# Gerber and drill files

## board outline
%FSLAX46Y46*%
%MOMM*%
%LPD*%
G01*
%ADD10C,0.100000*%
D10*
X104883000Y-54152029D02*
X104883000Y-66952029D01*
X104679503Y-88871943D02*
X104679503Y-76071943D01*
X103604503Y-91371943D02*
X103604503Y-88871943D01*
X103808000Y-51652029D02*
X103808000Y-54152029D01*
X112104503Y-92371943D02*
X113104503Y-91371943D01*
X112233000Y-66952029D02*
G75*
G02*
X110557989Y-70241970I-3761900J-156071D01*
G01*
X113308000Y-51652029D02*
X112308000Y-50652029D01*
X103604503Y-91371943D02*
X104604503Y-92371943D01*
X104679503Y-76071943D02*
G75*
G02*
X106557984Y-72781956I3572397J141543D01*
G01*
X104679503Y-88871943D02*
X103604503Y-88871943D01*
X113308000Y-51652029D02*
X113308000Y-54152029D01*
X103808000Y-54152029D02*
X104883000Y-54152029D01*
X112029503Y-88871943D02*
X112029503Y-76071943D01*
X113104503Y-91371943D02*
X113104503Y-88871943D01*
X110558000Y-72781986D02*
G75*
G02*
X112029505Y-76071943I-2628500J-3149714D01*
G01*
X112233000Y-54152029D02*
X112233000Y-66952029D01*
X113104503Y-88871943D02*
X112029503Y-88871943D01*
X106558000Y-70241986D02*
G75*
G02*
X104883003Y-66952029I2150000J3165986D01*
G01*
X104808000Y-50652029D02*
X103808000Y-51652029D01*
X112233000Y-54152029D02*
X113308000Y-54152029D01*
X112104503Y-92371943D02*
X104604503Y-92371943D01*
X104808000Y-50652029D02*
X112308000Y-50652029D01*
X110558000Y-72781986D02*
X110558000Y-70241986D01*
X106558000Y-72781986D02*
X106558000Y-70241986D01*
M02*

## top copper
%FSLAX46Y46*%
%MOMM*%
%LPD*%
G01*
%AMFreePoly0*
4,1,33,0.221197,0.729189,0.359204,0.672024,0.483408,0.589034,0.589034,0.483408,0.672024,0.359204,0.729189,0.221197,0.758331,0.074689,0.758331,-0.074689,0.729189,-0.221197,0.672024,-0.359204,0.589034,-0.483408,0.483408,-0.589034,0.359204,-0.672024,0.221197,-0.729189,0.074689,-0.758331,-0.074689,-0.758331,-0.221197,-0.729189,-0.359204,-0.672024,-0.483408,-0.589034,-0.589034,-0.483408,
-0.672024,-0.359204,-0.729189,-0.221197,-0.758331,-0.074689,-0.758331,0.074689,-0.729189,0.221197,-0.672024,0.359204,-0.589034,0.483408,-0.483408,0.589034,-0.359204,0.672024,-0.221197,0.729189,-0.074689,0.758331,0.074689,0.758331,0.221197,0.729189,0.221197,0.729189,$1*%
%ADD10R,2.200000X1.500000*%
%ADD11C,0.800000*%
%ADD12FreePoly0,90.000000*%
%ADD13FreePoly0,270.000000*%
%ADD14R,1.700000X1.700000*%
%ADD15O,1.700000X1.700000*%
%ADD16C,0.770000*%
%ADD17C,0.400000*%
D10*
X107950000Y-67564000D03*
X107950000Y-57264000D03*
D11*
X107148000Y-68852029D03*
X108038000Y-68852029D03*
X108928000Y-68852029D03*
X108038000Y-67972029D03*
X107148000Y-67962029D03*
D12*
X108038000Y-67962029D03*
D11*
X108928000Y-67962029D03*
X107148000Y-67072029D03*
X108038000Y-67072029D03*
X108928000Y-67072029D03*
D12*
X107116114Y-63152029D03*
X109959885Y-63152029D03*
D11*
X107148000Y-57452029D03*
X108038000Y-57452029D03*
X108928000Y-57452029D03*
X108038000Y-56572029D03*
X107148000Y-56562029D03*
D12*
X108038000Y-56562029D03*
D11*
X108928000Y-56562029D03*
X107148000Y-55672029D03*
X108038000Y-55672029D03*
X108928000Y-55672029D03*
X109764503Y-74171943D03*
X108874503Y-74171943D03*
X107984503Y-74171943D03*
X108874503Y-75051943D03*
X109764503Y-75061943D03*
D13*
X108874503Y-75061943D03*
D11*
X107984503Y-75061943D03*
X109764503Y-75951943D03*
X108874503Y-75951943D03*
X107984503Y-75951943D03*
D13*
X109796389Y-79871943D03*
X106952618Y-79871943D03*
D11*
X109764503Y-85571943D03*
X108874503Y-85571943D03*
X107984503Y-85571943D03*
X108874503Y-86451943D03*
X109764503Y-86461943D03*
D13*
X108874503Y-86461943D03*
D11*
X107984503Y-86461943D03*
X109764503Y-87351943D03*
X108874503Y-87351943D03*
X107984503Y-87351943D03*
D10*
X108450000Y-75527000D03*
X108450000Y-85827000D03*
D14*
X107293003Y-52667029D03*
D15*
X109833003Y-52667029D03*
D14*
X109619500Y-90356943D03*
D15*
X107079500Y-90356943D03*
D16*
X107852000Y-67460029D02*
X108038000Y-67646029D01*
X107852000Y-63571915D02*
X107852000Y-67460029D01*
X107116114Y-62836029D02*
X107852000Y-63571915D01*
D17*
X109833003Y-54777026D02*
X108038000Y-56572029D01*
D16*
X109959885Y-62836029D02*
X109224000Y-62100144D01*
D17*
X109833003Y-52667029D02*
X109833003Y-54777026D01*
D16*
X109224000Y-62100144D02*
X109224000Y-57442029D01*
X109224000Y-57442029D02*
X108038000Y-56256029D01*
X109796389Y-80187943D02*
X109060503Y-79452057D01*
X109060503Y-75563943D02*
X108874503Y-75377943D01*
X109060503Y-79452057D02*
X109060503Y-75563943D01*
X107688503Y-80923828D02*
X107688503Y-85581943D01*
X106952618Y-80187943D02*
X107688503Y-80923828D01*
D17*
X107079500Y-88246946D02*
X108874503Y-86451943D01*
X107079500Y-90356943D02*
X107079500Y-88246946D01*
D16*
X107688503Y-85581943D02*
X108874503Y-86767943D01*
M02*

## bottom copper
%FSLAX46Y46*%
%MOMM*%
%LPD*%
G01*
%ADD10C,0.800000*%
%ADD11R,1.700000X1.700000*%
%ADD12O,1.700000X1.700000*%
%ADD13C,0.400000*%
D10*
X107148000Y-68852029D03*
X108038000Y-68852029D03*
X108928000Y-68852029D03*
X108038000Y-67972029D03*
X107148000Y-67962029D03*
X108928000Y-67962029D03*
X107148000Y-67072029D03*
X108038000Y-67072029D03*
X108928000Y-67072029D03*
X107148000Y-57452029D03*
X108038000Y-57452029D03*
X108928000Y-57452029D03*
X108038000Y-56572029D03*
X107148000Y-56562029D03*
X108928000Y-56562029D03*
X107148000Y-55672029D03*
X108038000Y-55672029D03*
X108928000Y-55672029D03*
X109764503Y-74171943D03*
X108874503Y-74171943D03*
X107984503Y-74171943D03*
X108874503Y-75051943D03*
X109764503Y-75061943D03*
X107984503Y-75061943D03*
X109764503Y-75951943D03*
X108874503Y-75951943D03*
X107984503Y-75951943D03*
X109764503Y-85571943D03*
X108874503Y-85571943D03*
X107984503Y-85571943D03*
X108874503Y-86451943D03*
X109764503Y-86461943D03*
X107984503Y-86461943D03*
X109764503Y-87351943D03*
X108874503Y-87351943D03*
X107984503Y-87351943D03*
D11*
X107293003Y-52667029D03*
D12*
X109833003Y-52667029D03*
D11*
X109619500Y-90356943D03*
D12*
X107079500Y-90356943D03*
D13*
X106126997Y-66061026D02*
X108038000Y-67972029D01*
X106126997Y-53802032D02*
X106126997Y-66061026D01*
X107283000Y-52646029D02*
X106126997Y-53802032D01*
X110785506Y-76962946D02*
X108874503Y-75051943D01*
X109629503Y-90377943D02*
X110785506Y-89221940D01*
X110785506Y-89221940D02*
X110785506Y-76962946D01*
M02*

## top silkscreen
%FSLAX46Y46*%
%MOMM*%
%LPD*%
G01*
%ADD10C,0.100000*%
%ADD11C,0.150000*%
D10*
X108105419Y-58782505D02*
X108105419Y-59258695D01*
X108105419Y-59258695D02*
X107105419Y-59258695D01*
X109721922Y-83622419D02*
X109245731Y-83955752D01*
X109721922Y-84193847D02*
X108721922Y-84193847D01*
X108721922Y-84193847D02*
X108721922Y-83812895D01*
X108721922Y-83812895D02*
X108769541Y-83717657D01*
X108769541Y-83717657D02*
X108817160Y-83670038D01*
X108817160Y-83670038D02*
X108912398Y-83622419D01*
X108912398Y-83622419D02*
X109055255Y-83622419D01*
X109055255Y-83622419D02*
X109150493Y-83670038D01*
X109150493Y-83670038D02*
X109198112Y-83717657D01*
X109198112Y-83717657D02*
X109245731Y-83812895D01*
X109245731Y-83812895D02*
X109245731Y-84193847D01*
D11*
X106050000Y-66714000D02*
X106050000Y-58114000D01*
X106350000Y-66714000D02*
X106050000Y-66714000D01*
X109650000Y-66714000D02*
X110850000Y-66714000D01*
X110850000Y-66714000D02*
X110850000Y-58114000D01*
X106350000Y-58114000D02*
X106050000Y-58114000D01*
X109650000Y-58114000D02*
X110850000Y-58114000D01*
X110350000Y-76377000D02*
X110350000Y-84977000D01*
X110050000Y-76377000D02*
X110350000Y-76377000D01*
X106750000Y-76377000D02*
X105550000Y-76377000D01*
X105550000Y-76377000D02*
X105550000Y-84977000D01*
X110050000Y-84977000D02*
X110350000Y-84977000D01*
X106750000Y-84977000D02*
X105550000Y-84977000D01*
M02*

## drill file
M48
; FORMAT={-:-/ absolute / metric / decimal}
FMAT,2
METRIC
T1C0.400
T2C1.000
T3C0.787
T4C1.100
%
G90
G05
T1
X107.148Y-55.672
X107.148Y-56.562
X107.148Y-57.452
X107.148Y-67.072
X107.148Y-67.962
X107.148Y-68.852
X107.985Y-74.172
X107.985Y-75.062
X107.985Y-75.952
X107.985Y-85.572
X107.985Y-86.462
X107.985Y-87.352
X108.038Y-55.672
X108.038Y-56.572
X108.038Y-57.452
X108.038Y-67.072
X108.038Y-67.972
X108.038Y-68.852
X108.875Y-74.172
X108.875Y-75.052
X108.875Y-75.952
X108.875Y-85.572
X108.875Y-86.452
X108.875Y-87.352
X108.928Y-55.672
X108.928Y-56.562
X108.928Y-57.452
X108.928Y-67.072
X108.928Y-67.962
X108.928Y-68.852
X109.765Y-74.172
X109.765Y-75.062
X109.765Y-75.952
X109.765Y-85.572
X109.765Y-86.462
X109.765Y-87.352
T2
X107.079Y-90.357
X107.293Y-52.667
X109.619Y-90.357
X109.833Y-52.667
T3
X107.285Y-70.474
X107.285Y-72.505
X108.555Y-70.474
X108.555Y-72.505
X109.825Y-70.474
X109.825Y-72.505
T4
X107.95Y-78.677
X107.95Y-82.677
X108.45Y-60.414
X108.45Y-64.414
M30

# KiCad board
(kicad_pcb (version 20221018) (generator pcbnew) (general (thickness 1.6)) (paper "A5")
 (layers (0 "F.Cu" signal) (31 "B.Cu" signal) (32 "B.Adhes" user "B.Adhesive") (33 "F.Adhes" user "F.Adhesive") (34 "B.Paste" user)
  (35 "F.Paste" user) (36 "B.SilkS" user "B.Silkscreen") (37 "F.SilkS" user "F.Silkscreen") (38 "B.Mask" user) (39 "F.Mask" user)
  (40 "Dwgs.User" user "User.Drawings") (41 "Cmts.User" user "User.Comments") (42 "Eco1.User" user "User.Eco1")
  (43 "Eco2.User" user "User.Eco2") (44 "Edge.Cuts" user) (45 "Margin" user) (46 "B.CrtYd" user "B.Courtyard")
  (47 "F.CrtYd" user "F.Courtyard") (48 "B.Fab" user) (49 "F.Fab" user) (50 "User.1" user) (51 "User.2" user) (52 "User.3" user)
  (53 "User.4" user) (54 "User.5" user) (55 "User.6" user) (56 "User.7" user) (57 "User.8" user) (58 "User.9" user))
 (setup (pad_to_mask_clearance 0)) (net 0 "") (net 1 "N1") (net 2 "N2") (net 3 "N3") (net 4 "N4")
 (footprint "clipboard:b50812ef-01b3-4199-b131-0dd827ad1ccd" (layer "F.Cu") (at 110.95 68.339 90)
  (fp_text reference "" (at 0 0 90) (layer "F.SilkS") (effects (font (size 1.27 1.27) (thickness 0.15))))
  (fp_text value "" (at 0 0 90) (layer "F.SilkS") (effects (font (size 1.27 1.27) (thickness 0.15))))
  (fp_line (start 1.625 -4.9) (end 10.225 -4.9) (stroke (width 0.15) (type solid)) (layer "F.SilkS"))
  (fp_line (start 1.625 -4.6) (end 1.625 -4.9) (stroke (width 0.15) (type solid)) (layer "F.SilkS"))
  (fp_line (start 1.625 -1.3) (end 1.625 -0.1) (stroke (width 0.15) (type solid)) (layer "F.SilkS"))
  (fp_line (start 1.625 -0.1) (end 10.225 -0.1) (stroke (width 0.15) (type solid)) (layer "F.SilkS"))
  (fp_line (start 10.225 -4.6) (end 10.225 -4.9) (stroke (width 0.15) (type solid)) (layer "F.SilkS"))
  (fp_line (start 10.225 -1.3) (end 10.225 -0.1) (stroke (width 0.15) (type solid)) (layer "F.SilkS"))
  (pad "" np_thru_hole circle (at 3.925 -2.5 90) (size 1.1 1.1) (drill 1.1) (layers "F&B.Cu" "*.Mask"))
  (pad "" np_thru_hole circle (at 7.925 -2.5 90) (size 1.1 1.1) (drill 1.1) (layers "F&B.Cu" "*.Mask"))
  (pad "1" smd rect (at 0.775 -3 90) (size 1.5 2.2) (layers "F.Cu" "F.Paste" "F.Mask"))
  (pad "2" smd rect (at 11.075 -3 90) (size 1.5 2.2) (layers "F.Cu" "F.Paste" "F.Mask")))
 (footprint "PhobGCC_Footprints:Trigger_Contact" (layer "F.Cu") (at 108.538 63.152029 90)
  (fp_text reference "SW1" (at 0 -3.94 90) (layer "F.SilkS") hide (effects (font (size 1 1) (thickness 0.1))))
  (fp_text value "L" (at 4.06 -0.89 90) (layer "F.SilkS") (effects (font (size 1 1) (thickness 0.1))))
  (pad "1" thru_hole circle (at -5.7 -1.39 90) (size 0.8 0.8) (drill 0.4) (layers "*.Cu" "*.Mask") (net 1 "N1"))
  (pad "1" thru_hole circle (at -5.7 -0.5 90) (size 0.8 0.8) (drill 0.4) (layers "*.Cu" "*.Mask") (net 1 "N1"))
  (pad "1" thru_hole circle (at -5.7 0.39 90) (size 0.8 0.8) (drill 0.4) (layers "*.Cu" "*.Mask") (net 1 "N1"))
  (pad "1" thru_hole circle (at -4.82 -0.5 90) (size 0.8 0.8) (drill 0.4) (layers "*.Cu" "*.Mask") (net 1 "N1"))
  (pad "1" thru_hole circle (at -4.81 -1.39 90) (size 0.8 0.8) (drill 0.4) (layers "*.Cu" "*.Mask") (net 1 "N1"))
  (pad "1" smd custom (at -4.81 -0.5 90) (size 1.524 1.524) (layers "F.Cu" "F.Paste" "F.Mask") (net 1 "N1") (thermal_bridge_angle 45)
   (options (clearance outline) (anchor circle)) (primitives))
  (pad "1" thru_hole circle (at -4.81 0.39 90) (size 0.8 0.8) (drill 0.4) (layers "*.Cu" "*.Mask") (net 1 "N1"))
  (pad "1" thru_hole circle (at -3.92 -1.39 90) (size 0.8 0.8) (drill 0.4) (layers "*.Cu" "*.Mask") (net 1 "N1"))
  (pad "1" thru_hole circle (at -3.92 -0.5 90) (size 0.8 0.8) (drill 0.4) (layers "*.Cu" "*.Mask") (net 1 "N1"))
  (pad "1" thru_hole circle (at -3.92 0.39 90) (size 0.8 0.8) (drill 0.4) (layers "*.Cu" "*.Mask") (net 1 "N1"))
  (pad "1" smd custom (at 0 -1.421886 90) (size 1.524 1.524) (layers "F.Cu" "F.Paste" "F.Mask") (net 1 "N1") (thermal_bridge_angle 45)
   (options (clearance outline) (anchor circle)) (primitives))
  (pad "2" smd custom (at 0 1.421885 90) (size 1.524 1.524) (layers "F.Cu" "F.Paste" "F.Mask") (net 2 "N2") (thermal_bridge_angle 45)
   (options (clearance outline) (anchor circle)) (primitives))
  (pad "2" thru_hole circle (at 5.7 -1.39 90) (size 0.8 0.8) (drill 0.4) (layers "*.Cu" "*.Mask") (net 2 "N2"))
  (pad "2" thru_hole circle (at 5.7 -0.5 90) (size 0.8 0.8) (drill 0.4) (layers "*.Cu" "*.Mask") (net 2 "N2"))
  (pad "2" thru_hole circle (at 5.7 0.39 90) (size 0.8 0.8) (drill 0.4) (layers "*.Cu" "*.Mask") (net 2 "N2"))
  (pad "2" thru_hole circle (at 6.58 -0.5 90) (size 0.8 0.8) (drill 0.4) (layers "*.Cu" "*.Mask") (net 2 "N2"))
  (pad "2" thru_hole circle (at 6.59 -1.39 90) (size 0.8 0.8) (drill 0.4) (layers "*.Cu" "*.Mask") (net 2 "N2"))
  (pad "2" smd custom (at 6.59 -0.5 90) (size 1.524 1.524) (layers "F.Cu" "F.Paste" "F.Mask") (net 2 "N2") (thermal_bridge_angle 45)
   (options (clearance outline) (anchor circle)) (primitives))
  (pad "2" thru_hole circle (at 6.59 0.39 90) (size 0.8 0.8) (drill 0.4) (layers "*.Cu" "*.Mask") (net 2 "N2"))
  (pad "2" thru_hole circle (at 7.48 -1.39 90) (size 0.8 0.8) (drill 0.4) (layers "*.Cu" "*.Mask") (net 2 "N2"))
  (pad "2" thru_hole circle (at 7.48 -0.5 90) (size 0.8 0.8) (drill 0.4) (layers "*.Cu" "*.Mask") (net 2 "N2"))
  (pad "2" thru_hole circle (at 7.48 0.39 90) (size 0.8 0.8) (drill 0.4) (layers "*.Cu" "*.Mask") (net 2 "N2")))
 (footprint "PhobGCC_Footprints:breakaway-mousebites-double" (layer "F.Cu") (at 108.325 70.244093 180)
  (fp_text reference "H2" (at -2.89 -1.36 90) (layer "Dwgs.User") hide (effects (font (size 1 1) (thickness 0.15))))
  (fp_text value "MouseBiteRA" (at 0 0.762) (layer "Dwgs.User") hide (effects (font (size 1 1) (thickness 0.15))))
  (fp_line (start -2.233 -2.537893) (end -2.233 0.002107) (stroke (width 0.1) (type solid)) (layer "Edge.Cuts"))
  (fp_line (start 1.767 -2.537893) (end 1.767 0.002107) (stroke (width 0.1) (type solid)) (layer "Edge.Cuts"))
  (pad "" np_thru_hole circle (at -1.5 -2.26085) (size 0.7874 0.7874) (drill 0.7874) (layers "*.Cu" "*.Mask"))
  (pad "" np_thru_hole circle (at -1.5 -0.23 180) (size 0.7874 0.7874) (drill 0.7874) (layers "*.Cu" "*.Mask"))
  (pad "" np_thru_hole circle (at -0.23 -2.26085) (size 0.7874 0.7874) (drill 0.7874) (layers "*.Cu" "*.Mask"))
  (pad "" np_thru_hole circle (at -0.23 -0.23 180) (size 0.7874 0.7874) (drill 0.7874) (layers "*.Cu" "*.Mask"))
  (pad "" np_thru_hole circle (at 1.04 -2.26085) (size 0.7874 0.7874) (drill 0.7874) (layers "*.Cu" "*.Mask"))
  (pad "" np_thru_hole circle (at 1.04 -0.23 180) (size 0.7874 0.7874) (drill 0.7874) (layers "*.Cu" "*.Mask")))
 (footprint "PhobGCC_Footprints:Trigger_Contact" (layer "F.Cu") (at 108.374503 79.871943 -90)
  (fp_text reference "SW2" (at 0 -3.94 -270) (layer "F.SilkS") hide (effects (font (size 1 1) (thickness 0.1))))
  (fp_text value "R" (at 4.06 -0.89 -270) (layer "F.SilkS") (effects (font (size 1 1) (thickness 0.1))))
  (pad "1" thru_hole circle (at -5.7 -1.39 270) (size 0.8 0.8) (drill 0.4) (layers "*.Cu" "*.Mask") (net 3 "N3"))
  (pad "1" thru_hole circle (at -5.7 -0.5 270) (size 0.8 0.8) (drill 0.4) (layers "*.Cu" "*.Mask") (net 3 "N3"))
  (pad "1" thru_hole circle (at -5.7 0.39 270) (size 0.8 0.8) (drill 0.4) (layers "*.Cu" "*.Mask") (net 3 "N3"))
  (pad "1" thru_hole circle (at -4.82 -0.5 270) (size 0.8 0.8) (drill 0.4) (layers "*.Cu" "*.Mask") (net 3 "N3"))
  (pad "1" thru_hole circle (at -4.81 -1.39 270) (size 0.8 0.8) (drill 0.4) (layers "*.Cu" "*.Mask") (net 3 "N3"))
  (pad "1" smd custom (at -4.81 -0.5 270) (size 1.524 1.524) (layers "F.Cu" "F.Paste" "F.Mask") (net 3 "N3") (thermal_bridge_angle 45)
   (options (clearance outline) (anchor circle)) (primitives))
  (pad "1" thru_hole circle (at -4.81 0.39 270) (size 0.8 0.8) (drill 0.4) (layers "*.Cu" "*.Mask") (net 3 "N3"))
  (pad "1" thru_hole circle (at -3.92 -1.39 270) (size 0.8 0.8) (drill 0.4) (layers "*.Cu" "*.Mask") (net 3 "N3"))
  (pad "1" thru_hole circle (at -3.92 -0.5 270) (size 0.8 0.8) (drill 0.4) (layers "*.Cu" "*.Mask") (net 3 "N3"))
  (pad "1" thru_hole circle (at -3.92 0.39 270) (size 0.8 0.8) (drill 0.4) (layers "*.Cu" "*.Mask") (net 3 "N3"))
  (pad "1" smd custom (at 0 -1.421886 270) (size 1.524 1.524) (layers "F.Cu" "F.Paste" "F.Mask") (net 3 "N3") (thermal_bridge_angle 45)
   (options (clearance outline) (anchor circle)) (primitives))
  (pad "2" smd custom (at 0 1.421885 270) (size 1.524 1.524) (layers "F.Cu" "F.Paste" "F.Mask") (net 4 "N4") (thermal_bridge_angle 45)
   (options (clearance outline) (anchor circle)) (primitives))
  (pad "2" thru_hole circle (at 5.7 -1.39 270) (size 0.8 0.8) (drill 0.4) (layers "*.Cu" "*.Mask") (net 4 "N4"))
  (pad "2" thru_hole circle (at 5.7 -0.5 270) (size 0.8 0.8) (drill 0.4) (layers "*.Cu" "*.Mask") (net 4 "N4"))
  (pad "2" thru_hole circle (at 5.7 0.39 270) (size 0.8 0.8) (drill 0.4) (layers "*.Cu" "*.Mask") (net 4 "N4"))
  (pad "2" thru_hole circle (at 6.58 -0.5 270) (size 0.8 0.8) (drill 0.4) (layers "*.Cu" "*.Mask") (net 4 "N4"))
  (pad "2" thru_hole circle (at 6.59 -1.39 270) (size 0.8 0.8) (drill 0.4) (layers "*.Cu" "*.Mask") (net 4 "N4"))
  (pad "2" smd custom (at 6.59 -0.5 270) (size 1.524 1.524) (layers "F.Cu" "F.Paste" "F.Mask") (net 4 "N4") (thermal_bridge_angle 45)
   (options (clearance outline) (anchor circle)) (primitives))
  (pad "2" thru_hole circle (at 6.59 0.39 270) (size 0.8 0.8) (drill 0.4) (layers "*.Cu" "*.Mask") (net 4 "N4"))
  (pad "2" thru_hole circle (at 7.48 -1.39 270) (size 0.8 0.8) (drill 0.4) (layers "*.Cu" "*.Mask") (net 4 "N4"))
  (pad "2" thru_hole circle (at 7.48 -0.5 270) (size 0.8 0.8) (drill 0.4) (layers "*.Cu" "*.Mask") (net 4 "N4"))
  (pad "2" thru_hole circle (at 7.48 0.39 270) (size 0.8 0.8) (drill 0.4) (layers "*.Cu" "*.Mask") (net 4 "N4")))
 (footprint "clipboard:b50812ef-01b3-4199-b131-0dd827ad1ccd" (layer "F.Cu") (at 105.45 74.752 -90)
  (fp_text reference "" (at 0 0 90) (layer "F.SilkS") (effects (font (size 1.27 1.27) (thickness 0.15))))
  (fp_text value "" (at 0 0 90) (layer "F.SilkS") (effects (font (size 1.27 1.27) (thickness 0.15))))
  (fp_line (start 1.625 -4.9) (end 10.225 -4.9) (stroke (width 0.15) (type solid)) (layer "F.SilkS"))
  (fp_line (start 1.625 -4.6) (end 1.625 -4.9) (stroke (width 0.15) (type solid)) (layer "F.SilkS"))
  (fp_line (start 1.625 -1.3) (end 1.625 -0.1) (stroke (width 0.15) (type solid)) (layer "F.SilkS"))
  (fp_line (start 1.625 -0.1) (end 10.225 -0.1) (stroke (width 0.15) (type solid)) (layer "F.SilkS"))
  (fp_line (start 10.225 -4.6) (end 10.225 -4.9) (stroke (width 0.15) (type solid)) (layer "F.SilkS"))
  (fp_line (start 10.225 -1.3) (end 10.225 -0.1) (stroke (width 0.15) (type solid)) (layer "F.SilkS"))
  (pad "" np_thru_hole circle (at 3.925 -2.5 270) (size 1.1 1.1) (drill 1.1) (layers "F&B.Cu" "*.Mask"))
  (pad "" np_thru_hole circle (at 7.925 -2.5 270) (size 1.1 1.1) (drill 1.1) (layers "F&B.Cu" "*.Mask"))
  (pad "1" smd rect (at 0.775 -3 270) (size 1.5 2.2) (layers "F.Cu" "F.Paste" "F.Mask"))
  (pad "2" smd rect (at 11.075 -3 270) (size 1.5 2.2) (layers "F.Cu" "F.Paste" "F.Mask")))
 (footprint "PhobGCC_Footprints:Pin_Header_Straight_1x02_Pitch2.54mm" (layer "B.Cu") (at 107.293003 52.667029 -90)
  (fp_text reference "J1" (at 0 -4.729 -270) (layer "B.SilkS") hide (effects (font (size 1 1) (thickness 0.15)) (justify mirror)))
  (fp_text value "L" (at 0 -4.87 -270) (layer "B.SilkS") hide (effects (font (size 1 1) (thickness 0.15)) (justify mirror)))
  (pad "1" thru_hole rect (at 0 0 270) (size 1.7 1.7) (drill 1) (layers "*.Cu" "*.Mask") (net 1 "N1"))
  (pad "2" thru_hole oval (at 0 -2.54 270) (size 1.7 1.7) (drill 1) (layers "*.Cu" "*.Mask") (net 2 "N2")))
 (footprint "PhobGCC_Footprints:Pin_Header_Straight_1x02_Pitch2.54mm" (layer "B.Cu") (at 109.6195 90.356943 90)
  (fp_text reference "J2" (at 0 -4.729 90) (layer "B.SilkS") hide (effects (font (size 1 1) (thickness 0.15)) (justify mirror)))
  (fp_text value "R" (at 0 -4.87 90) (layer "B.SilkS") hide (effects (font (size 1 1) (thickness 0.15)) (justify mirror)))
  (pad "1" thru_hole rect (at 0 0 90) (size 1.7 1.7) (drill 1) (layers "*.Cu" "*.Mask") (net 3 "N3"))
  (pad "2" thru_hole oval (at 0 -2.54 90) (size 1.7 1.7) (drill 1) (layers "*.Cu" "*.Mask") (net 4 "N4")))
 (gr_line (start 104.883 54.152029) (end 104.883 66.952029) (stroke (width 0.1) (type solid)) (layer "Edge.Cuts"))
 (gr_line (start 104.679503 88.871943) (end 104.679503 76.071943) (stroke (width 0.1) (type solid)) (layer "Edge.Cuts"))
 (gr_line (start 103.604503 91.371943) (end 103.604503 88.871943) (stroke (width 0.1) (type solid)) (layer "Edge.Cuts"))
 (gr_line (start 103.808 51.652029) (end 103.808 54.152029) (stroke (width 0.1) (type solid)) (layer "Edge.Cuts"))
 (gr_line (start 112.104503 92.371943) (end 113.104503 91.371943) (stroke (width 0.1) (type solid)) (layer "Edge.Cuts"))
 (gr_arc (start 112.233 66.952029) (mid 111.826403 68.816395) (end 110.558 70.241986) (stroke (width 0.1) (type solid)) (layer "Edge.Cuts"))
 (gr_line (start 113.308 51.652029) (end 112.308 50.652029) (stroke (width 0.1) (type solid)) (layer "Edge.Cuts"))
 (gr_line (start 103.604503 91.371943) (end 104.604503 92.371943) (stroke (width 0.1) (type solid)) (layer "Edge.Cuts"))
 (gr_arc (start 104.679503 76.071943) (mid 105.14715 74.157693) (end 106.558 72.781986) (stroke (width 0.1) (type solid))
  (layer "Edge.Cuts"))
 (gr_line (start 104.679503 88.871943) (end 103.604503 88.871943) (stroke (width 0.1) (type solid)) (layer "Edge.Cuts"))
 (gr_line (start 113.308 51.652029) (end 113.308 54.152029) (stroke (width 0.1) (type solid)) (layer "Edge.Cuts"))
 (gr_line (start 103.808 54.152029) (end 104.883 54.152029) (stroke (width 0.1) (type solid)) (layer "Edge.Cuts"))
 (gr_line (start 112.029503 88.871943) (end 112.029503 76.071943) (stroke (width 0.1) (type solid)) (layer "Edge.Cuts"))
 (gr_line (start 113.104503 91.371943) (end 113.104503 88.871943) (stroke (width 0.1) (type solid)) (layer "Edge.Cuts"))
 (gr_arc (start 110.558 72.781986) (mid 111.674383 74.256719) (end 112.029503 76.071943) (stroke (width 0.1) (type solid))
  (layer "Edge.Cuts"))
 (gr_line (start 112.233 54.152029) (end 112.233 66.952029) (stroke (width 0.1) (type solid)) (layer "Edge.Cuts"))
 (gr_line (start 113.104503 88.871943) (end 112.029503 88.871943) (stroke (width 0.1) (type solid)) (layer "Edge.Cuts"))
 (gr_arc (start 106.558 70.241986) (mid 105.297554 68.812335) (end 104.883 66.952029) (stroke (width 0.1) (type solid)) (layer "Edge.Cuts"))
 (gr_line (start 104.808 50.652029) (end 103.808 51.652029) (stroke (width 0.1) (type solid)) (layer "Edge.Cuts"))
 (gr_line (start 112.233 54.152029) (end 113.308 54.152029) (stroke (width 0.1) (type solid)) (layer "Edge.Cuts"))
 (gr_line (start 112.104503 92.371943) (end 104.604503 92.371943) (stroke (width 0.1) (type solid)) (layer "Edge.Cuts"))
 (gr_line (start 104.808 50.652029) (end 112.308 50.652029) (stroke (width 0.1) (type solid)) (layer "Edge.Cuts"))
 (segment (start 107.852 67.460029) (end 108.038 67.646029) (width 0.77) (layer "F.Cu") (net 1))
 (segment (start 107.852 63.571915) (end 107.852 67.460029) (width 0.77) (layer "F.Cu") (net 1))
 (segment (start 107.116114 62.836029) (end 107.852 63.571915) (width 0.77) (layer "F.Cu") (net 1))
 (segment (start 106.126997 66.061026) (end 108.038 67.972029) (width 0.4) (layer "B.Cu") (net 1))
 (segment (start 106.126997 53.802032) (end 106.126997 66.061026) (width 0.4) (layer "B.Cu") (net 1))
 (segment (start 107.283 52.646029) (end 106.126997 53.802032) (width 0.4) (layer "B.Cu") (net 1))
 (segment (start 109.833003 54.777026) (end 108.038 56.572029) (width 0.4) (layer "F.Cu") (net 2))
 (segment (start 109.959885 62.836029) (end 109.224 62.100144) (width 0.77) (layer "F.Cu") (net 2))
 (segment (start 109.833003 52.667029) (end 109.833003 54.777026) (width 0.4) (layer "F.Cu") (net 2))
 (segment (start 109.224 62.100144) (end 109.224 57.442029) (width 0.77) (layer "F.Cu") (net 2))
 (segment (start 109.224 57.442029) (end 108.038 56.256029) (width 0.77) (layer "F.Cu") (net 2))
 (segment (start 109.796389 80.187943) (end 109.060503 79.452057) (width 0.77) (layer "F.Cu") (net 3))
 (segment (start 109.060503 75.563943) (end 108.874503 75.377943) (width 0.77) (layer "F.Cu") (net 3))
 (segment (start 109.060503 79.452057) (end 109.060503 75.563943) (width 0.77) (layer "F.Cu") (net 3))
 (segment (start 110.785506 76.962946) (end 108.874503 75.051943) (width 0.4) (layer "B.Cu") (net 3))
 (segment (start 109.629503 90.377943) (end 110.785506 89.22194) (width 0.4) (layer "B.Cu") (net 3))
 (segment (start 110.785506 89.22194) (end 110.785506 76.962946) (width 0.4) (layer "B.Cu") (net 3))
 (segment (start 107.688503 80.923828) (end 107.688503 85.581943) (width 0.77) (layer "F.Cu") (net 4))
 (segment (start 106.952618 80.187943) (end 107.688503 80.923828) (width 0.77) (layer "F.Cu") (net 4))
 (segment (start 107.0795 88.246946) (end 108.874503 86.451943) (width 0.4) (layer "F.Cu") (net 4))
 (segment (start 107.0795 90.356943) (end 107.0795 88.246946) (width 0.4) (layer "F.Cu") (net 4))
 (segment (start 107.688503 85.581943) (end 108.874503 86.767943) (width 0.77) (layer "F.Cu") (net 4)))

